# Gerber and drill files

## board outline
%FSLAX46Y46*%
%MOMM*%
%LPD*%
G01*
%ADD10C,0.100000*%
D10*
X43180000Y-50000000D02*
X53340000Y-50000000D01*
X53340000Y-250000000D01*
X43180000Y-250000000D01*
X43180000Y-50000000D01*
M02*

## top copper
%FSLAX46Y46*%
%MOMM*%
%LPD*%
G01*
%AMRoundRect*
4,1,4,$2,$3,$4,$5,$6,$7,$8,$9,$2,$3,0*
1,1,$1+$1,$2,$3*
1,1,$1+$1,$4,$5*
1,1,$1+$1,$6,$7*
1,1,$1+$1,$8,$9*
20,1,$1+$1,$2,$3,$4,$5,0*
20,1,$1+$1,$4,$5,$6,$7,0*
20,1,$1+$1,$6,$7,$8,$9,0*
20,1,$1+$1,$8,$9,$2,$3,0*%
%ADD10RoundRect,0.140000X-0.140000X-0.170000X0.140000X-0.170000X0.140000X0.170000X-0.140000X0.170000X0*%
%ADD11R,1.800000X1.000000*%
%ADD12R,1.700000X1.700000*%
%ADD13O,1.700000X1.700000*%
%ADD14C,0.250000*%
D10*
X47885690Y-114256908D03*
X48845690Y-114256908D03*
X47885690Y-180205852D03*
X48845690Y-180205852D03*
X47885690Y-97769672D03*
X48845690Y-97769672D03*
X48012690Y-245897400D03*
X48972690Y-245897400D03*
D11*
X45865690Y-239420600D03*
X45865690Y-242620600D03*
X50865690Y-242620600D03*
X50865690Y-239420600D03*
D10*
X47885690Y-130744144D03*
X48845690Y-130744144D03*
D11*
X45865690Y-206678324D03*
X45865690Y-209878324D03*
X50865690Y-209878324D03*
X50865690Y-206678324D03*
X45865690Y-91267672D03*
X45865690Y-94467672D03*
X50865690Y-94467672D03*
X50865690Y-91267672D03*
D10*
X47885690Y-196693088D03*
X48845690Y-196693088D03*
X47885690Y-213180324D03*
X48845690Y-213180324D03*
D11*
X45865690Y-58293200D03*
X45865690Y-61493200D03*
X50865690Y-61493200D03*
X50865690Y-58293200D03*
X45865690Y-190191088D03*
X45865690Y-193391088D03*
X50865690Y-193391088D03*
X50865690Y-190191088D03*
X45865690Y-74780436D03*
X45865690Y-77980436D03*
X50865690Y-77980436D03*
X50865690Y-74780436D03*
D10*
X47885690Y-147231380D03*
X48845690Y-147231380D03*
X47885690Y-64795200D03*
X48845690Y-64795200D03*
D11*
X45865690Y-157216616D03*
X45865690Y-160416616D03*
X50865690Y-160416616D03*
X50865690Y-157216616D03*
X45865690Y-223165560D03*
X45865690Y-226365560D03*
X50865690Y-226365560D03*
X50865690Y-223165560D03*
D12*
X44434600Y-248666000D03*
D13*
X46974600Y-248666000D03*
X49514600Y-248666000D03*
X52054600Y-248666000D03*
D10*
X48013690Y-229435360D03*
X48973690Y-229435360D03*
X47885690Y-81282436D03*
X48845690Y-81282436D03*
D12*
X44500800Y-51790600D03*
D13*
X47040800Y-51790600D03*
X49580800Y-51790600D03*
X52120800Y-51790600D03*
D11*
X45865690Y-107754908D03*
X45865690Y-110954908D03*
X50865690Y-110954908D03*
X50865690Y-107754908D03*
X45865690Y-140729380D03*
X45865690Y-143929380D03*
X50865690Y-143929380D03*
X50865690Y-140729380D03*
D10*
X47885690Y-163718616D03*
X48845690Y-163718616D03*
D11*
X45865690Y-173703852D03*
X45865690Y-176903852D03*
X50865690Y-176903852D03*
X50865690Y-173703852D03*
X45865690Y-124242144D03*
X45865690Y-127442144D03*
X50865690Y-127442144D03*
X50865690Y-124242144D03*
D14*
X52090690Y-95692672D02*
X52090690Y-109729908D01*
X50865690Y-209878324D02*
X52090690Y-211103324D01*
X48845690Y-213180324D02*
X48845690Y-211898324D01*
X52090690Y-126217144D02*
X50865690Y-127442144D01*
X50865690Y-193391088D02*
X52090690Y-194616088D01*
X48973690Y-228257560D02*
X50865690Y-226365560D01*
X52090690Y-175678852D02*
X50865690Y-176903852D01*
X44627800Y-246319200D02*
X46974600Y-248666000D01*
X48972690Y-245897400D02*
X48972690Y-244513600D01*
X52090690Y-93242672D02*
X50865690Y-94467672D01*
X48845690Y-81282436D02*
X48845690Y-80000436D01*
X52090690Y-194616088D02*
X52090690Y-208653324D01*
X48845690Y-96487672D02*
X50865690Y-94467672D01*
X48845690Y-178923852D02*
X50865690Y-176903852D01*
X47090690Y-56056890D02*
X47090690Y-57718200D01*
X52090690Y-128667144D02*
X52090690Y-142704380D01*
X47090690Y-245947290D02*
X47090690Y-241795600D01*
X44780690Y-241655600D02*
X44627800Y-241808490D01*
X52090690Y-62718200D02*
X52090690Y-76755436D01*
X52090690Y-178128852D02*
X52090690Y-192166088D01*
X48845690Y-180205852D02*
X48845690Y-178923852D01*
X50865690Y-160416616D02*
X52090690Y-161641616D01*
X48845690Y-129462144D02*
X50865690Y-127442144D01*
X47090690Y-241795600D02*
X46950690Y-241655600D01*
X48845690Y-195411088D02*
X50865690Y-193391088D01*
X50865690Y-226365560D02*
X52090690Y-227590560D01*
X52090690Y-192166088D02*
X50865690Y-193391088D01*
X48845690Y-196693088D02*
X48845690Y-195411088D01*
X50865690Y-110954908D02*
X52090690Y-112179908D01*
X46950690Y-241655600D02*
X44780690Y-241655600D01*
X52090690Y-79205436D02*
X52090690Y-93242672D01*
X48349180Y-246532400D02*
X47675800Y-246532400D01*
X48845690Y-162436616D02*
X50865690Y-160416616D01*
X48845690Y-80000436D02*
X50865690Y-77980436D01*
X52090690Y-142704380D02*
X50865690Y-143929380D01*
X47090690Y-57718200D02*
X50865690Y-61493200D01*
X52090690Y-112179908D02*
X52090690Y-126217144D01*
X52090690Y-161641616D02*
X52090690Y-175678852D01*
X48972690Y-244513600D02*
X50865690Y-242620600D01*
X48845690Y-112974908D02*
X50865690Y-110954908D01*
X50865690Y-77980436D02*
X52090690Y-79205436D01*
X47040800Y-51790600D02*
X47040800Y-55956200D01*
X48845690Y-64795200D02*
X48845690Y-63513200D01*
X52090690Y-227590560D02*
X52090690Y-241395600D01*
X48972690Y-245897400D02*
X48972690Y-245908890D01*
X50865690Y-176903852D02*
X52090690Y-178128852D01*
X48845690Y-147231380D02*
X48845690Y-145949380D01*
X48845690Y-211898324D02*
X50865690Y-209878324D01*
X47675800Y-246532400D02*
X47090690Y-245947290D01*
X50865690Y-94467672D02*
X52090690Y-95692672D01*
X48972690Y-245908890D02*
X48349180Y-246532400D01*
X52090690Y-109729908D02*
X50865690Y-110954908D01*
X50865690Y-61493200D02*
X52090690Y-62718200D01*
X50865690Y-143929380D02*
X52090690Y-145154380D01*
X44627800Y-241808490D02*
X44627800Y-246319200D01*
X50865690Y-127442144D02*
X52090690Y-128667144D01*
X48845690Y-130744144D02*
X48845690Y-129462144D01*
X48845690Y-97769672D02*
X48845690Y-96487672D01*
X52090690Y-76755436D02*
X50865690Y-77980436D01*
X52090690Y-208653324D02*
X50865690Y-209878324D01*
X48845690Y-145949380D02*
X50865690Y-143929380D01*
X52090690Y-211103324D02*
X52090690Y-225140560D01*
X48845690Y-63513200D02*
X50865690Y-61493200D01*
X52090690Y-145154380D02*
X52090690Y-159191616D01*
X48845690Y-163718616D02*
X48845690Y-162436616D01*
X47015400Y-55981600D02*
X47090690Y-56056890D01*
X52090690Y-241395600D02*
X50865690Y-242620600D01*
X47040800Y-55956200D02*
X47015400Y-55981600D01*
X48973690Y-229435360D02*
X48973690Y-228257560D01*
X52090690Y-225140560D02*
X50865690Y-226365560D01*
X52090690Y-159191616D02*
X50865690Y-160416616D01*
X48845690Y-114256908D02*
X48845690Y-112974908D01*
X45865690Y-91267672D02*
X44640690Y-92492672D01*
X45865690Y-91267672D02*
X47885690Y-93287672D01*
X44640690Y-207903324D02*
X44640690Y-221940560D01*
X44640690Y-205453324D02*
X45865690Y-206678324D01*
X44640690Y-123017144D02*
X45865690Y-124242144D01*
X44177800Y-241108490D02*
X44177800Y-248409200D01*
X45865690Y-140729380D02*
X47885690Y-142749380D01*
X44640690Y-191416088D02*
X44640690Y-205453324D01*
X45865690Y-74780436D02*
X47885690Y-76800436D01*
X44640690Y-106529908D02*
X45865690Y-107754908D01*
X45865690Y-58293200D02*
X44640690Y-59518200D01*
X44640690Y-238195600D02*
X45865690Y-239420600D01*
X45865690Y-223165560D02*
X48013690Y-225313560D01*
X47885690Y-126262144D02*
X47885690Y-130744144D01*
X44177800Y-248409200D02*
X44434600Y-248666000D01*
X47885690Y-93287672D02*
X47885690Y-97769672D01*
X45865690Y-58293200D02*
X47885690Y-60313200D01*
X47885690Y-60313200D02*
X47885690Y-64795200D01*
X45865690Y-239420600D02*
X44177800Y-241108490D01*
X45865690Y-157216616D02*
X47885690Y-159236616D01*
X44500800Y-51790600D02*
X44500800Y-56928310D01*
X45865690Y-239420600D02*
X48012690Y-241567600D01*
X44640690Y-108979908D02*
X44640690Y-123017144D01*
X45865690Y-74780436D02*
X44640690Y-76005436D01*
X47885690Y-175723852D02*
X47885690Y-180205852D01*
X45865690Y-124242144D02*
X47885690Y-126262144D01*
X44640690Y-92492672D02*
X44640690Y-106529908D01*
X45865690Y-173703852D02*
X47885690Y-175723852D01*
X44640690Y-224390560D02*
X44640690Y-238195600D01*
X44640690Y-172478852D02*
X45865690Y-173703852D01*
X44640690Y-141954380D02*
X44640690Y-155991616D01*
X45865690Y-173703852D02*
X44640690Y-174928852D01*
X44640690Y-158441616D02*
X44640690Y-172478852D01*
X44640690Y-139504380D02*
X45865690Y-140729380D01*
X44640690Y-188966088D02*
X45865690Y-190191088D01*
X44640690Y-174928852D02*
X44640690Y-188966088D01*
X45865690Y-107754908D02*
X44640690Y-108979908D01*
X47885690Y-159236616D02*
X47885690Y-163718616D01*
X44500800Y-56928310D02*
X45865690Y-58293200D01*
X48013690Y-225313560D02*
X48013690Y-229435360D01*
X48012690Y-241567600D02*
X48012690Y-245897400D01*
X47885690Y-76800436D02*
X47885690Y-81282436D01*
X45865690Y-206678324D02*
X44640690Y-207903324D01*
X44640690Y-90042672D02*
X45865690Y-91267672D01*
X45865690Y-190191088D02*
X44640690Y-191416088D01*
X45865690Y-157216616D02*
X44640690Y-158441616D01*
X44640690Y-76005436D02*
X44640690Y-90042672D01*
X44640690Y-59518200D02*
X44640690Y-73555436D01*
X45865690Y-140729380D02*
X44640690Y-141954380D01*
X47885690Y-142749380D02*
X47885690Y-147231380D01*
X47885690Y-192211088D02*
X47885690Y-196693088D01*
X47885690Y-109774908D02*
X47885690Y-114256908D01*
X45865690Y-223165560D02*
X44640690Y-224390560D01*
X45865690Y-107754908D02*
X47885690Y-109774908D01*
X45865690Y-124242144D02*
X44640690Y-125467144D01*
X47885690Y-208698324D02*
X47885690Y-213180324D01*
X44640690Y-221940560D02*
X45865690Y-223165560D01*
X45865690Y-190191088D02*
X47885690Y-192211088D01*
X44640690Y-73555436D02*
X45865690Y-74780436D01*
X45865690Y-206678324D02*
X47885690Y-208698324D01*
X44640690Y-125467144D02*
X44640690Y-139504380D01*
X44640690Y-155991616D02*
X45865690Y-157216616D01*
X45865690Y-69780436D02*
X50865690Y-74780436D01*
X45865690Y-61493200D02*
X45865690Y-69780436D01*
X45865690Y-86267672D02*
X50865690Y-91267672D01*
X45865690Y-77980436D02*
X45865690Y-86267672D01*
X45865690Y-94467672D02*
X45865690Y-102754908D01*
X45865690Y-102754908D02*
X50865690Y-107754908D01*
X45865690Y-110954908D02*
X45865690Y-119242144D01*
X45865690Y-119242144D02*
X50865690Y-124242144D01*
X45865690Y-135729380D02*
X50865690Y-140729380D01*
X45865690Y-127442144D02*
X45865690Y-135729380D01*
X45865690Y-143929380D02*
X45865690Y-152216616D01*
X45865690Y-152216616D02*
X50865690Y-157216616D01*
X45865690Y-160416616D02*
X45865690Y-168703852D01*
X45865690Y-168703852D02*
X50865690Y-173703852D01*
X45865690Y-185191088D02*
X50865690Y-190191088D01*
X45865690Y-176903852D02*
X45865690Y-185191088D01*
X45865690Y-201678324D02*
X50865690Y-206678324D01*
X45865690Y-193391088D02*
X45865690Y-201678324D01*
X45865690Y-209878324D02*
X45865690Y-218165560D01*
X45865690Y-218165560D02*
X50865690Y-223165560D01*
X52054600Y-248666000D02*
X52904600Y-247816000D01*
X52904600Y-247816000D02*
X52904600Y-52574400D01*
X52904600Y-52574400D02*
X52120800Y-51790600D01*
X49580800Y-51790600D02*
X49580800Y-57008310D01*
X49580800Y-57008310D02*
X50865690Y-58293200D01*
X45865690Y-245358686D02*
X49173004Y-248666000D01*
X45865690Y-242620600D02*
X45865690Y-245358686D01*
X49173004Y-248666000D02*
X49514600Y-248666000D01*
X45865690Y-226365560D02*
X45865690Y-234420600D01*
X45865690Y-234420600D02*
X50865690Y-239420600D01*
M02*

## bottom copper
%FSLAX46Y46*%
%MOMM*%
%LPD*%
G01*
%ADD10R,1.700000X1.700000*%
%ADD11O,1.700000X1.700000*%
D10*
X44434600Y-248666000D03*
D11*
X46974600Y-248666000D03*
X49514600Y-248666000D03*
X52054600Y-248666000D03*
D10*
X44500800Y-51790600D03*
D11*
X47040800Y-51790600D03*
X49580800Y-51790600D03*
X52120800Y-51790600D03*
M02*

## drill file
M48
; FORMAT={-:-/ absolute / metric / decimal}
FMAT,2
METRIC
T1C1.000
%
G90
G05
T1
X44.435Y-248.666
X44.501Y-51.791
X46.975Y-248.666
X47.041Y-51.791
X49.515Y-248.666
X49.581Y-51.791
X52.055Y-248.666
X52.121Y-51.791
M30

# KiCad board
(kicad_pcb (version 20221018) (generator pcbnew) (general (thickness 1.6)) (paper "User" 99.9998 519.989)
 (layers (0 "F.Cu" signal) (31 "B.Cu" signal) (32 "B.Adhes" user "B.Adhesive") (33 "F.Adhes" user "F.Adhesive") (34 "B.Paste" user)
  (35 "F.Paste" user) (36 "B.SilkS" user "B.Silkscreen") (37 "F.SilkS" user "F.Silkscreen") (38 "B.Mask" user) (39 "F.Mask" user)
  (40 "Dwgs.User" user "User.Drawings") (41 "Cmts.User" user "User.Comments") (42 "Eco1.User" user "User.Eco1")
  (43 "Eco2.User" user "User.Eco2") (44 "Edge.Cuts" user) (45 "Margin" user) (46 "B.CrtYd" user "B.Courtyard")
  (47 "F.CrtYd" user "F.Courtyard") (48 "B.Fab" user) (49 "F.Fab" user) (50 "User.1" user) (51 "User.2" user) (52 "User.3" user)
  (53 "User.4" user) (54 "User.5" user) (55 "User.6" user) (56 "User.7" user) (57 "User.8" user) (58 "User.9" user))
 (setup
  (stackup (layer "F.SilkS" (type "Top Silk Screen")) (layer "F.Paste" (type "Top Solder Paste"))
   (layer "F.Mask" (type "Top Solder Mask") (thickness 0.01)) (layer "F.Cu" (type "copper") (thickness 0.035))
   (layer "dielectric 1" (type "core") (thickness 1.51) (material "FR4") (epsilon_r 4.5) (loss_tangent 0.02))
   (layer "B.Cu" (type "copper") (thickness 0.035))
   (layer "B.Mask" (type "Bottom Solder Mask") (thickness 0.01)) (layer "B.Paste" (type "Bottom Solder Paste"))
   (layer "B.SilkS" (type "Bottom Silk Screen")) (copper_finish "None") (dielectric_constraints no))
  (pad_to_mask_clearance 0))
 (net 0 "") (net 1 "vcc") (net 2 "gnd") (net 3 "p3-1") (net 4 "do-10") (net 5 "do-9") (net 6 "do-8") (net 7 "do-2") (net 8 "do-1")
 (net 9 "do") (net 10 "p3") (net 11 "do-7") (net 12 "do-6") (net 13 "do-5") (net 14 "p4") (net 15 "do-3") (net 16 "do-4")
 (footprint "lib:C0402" (layer "F.Cu") (at 48.36569 114.256908)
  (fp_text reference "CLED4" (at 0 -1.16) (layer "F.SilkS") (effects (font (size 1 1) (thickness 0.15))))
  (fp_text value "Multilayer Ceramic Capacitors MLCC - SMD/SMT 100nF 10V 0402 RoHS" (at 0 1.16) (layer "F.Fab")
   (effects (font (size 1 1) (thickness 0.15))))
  (pad "1" smd roundrect (at -0.48 0) (size 0.56 0.62) (layers "F.Cu" "F.Paste" "F.Mask") (roundrect_rratio 0.25) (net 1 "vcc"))
  (pad "2" smd roundrect (at 0.48 0) (size 0.56 0.62) (layers "F.Cu" "F.Paste" "F.Mask") (roundrect_rratio 0.25) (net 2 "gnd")))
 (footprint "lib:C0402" (layer "F.Cu") (at 48.36569 180.205852)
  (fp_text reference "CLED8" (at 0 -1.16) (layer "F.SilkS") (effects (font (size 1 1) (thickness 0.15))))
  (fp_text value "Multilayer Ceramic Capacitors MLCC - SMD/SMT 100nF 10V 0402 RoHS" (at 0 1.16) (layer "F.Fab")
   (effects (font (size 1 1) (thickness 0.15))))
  (pad "1" smd roundrect (at -0.48 0) (size 0.56 0.62) (layers "F.Cu" "F.Paste" "F.Mask") (roundrect_rratio 0.25) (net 1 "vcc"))
  (pad "2" smd roundrect (at 0.48 0) (size 0.56 0.62) (layers "F.Cu" "F.Paste" "F.Mask") (roundrect_rratio 0.25) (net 2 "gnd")))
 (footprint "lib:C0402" (layer "F.Cu") (at 48.36569 97.769672)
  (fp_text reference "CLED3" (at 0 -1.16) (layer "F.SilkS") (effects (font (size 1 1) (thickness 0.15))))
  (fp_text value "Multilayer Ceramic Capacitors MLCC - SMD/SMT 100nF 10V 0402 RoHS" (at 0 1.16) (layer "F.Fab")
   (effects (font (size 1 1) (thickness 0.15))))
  (pad "1" smd roundrect (at -0.48 0) (size 0.56 0.62) (layers "F.Cu" "F.Paste" "F.Mask") (roundrect_rratio 0.25) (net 1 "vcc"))
  (pad "2" smd roundrect (at 0.48 0) (size 0.56 0.62) (layers "F.Cu" "F.Paste" "F.Mask") (roundrect_rratio 0.25) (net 2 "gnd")))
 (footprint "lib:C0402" (layer "F.Cu") (at 48.49269 245.8974)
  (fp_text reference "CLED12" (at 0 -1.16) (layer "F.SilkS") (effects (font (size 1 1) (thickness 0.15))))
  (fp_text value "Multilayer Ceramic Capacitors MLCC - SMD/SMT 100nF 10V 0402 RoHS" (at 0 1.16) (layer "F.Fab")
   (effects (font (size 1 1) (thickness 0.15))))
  (pad "1" smd roundrect (at -0.48 0) (size 0.56 0.62) (layers "F.Cu" "F.Paste" "F.Mask") (roundrect_rratio 0.25) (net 1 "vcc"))
  (pad "2" smd roundrect (at 0.48 0) (size 0.56 0.62) (layers "F.Cu" "F.Paste" "F.Mask") (roundrect_rratio 0.25) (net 2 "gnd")))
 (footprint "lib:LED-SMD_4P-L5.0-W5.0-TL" (layer "F.Cu") (at 48.36569 241.0206)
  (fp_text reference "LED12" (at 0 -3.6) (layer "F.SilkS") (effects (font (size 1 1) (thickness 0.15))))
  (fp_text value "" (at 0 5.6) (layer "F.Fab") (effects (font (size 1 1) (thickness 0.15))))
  (pad "1" smd rect (at -2.5 -1.6 180) (size 1.8 1) (layers "F.Cu" "F.Paste" "F.Mask") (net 1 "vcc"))
  (pad "2" smd rect (at -2.5 1.6 180) (size 1.8 1) (layers "F.Cu" "F.Paste" "F.Mask") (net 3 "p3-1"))
  (pad "3" smd rect (at 2.5 1.6 180) (size 1.8 1) (layers "F.Cu" "F.Paste" "F.Mask") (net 2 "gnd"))
  (pad "4" smd rect (at 2.5 -1.6 180) (size 1.8 1) (layers "F.Cu" "F.Paste" "F.Mask") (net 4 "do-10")))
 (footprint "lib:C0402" (layer "F.Cu") (at 48.36569 130.744144)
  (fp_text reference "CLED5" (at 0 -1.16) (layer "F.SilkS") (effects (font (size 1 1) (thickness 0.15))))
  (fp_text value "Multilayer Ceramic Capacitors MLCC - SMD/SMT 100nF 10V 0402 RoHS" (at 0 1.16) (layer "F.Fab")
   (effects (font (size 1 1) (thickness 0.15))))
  (pad "1" smd roundrect (at -0.48 0) (size 0.56 0.62) (layers "F.Cu" "F.Paste" "F.Mask") (roundrect_rratio 0.25) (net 1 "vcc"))
  (pad "2" smd roundrect (at 0.48 0) (size 0.56 0.62) (layers "F.Cu" "F.Paste" "F.Mask") (roundrect_rratio 0.25) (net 2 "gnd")))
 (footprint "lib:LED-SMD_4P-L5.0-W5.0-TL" (layer "F.Cu") (at 48.36569 208.278324)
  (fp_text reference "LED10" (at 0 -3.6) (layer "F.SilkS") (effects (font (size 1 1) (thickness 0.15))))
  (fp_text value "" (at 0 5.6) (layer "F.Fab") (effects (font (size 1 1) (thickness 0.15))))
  (pad "1" smd rect (at -2.5 -1.6 180) (size 1.8 1) (layers "F.Cu" "F.Paste" "F.Mask") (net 1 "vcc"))
  (pad "2" smd rect (at -2.5 1.6 180) (size 1.8 1) (layers "F.Cu" "F.Paste" "F.Mask") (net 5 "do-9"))
  (pad "3" smd rect (at 2.5 1.6 180) (size 1.8 1) (layers "F.Cu" "F.Paste" "F.Mask") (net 2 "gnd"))
  (pad "4" smd rect (at 2.5 -1.6 180) (size 1.8 1) (layers "F.Cu" "F.Paste" "F.Mask") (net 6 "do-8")))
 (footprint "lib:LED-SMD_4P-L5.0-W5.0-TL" (layer "F.Cu") (at 48.36569 92.867672)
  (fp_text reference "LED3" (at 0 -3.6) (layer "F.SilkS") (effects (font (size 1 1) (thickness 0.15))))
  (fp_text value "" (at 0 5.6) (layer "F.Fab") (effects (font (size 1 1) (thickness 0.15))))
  (pad "1" smd rect (at -2.5 -1.6 180) (size 1.8 1) (layers "F.Cu" "F.Paste" "F.Mask") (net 1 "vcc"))
  (pad "2" smd rect (at -2.5 1.6 180) (size 1.8 1) (layers "F.Cu" "F.Paste" "F.Mask") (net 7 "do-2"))
  (pad "3" smd rect (at 2.5 1.6 180) (size 1.8 1) (layers "F.Cu" "F.Paste" "F.Mask") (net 2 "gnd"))
  (pad "4" smd rect (at 2.5 -1.6 180) (size 1.8 1) (layers "F.Cu" "F.Paste" "F.Mask") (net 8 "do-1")))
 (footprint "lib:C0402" (layer "F.Cu") (at 48.36569 196.693088)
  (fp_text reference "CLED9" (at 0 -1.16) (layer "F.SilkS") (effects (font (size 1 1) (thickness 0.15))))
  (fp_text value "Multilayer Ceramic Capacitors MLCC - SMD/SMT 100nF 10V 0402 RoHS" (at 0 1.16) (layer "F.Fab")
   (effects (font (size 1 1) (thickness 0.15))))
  (pad "1" smd roundrect (at -0.48 0) (size 0.56 0.62) (layers "F.Cu" "F.Paste" "F.Mask") (roundrect_rratio 0.25) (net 1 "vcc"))
  (pad "2" smd roundrect (at 0.48 0) (size 0.56 0.62) (layers "F.Cu" "F.Paste" "F.Mask") (roundrect_rratio 0.25) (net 2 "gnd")))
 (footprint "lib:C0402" (layer "F.Cu") (at 48.36569 213.180324)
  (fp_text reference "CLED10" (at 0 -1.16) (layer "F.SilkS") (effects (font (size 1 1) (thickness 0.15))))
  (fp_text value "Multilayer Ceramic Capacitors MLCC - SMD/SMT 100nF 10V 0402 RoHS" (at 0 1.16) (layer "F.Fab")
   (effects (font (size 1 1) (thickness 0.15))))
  (pad "1" smd roundrect (at -0.48 0) (size 0.56 0.62) (layers "F.Cu" "F.Paste" "F.Mask") (roundrect_rratio 0.25) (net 1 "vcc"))
  (pad "2" smd roundrect (at 0.48 0) (size 0.56 0.62) (layers "F.Cu" "F.Paste" "F.Mask") (roundrect_rratio 0.25) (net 2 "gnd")))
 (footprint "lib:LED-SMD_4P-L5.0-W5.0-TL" (layer "F.Cu") (at 48.36569 59.8932)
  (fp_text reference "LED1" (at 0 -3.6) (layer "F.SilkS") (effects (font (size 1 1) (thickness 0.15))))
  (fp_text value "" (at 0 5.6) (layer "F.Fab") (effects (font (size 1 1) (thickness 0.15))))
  (pad "1" smd rect (at -2.5 -1.6 180) (size 1.8 1) (layers "F.Cu" "F.Paste" "F.Mask") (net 1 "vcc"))
  (pad "2" smd rect (at -2.5 1.6 180) (size 1.8 1) (layers "F.Cu" "F.Paste" "F.Mask") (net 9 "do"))
  (pad "3" smd rect (at 2.5 1.6 180) (size 1.8 1) (layers "F.Cu" "F.Paste" "F.Mask") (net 2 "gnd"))
  (pad "4" smd rect (at 2.5 -1.6 180) (size 1.8 1) (layers "F.Cu" "F.Paste" "F.Mask") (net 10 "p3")))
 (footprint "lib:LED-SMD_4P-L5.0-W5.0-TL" (layer "F.Cu") (at 48.36569 191.791088)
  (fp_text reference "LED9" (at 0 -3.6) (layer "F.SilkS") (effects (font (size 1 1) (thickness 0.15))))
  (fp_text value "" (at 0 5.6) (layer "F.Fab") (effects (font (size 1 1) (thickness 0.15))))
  (pad "1" smd rect (at -2.5 -1.6 180) (size 1.8 1) (layers "F.Cu" "F.Paste" "F.Mask") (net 1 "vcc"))
  (pad "2" smd rect (at -2.5 1.6 180) (size 1.8 1) (layers "F.Cu" "F.Paste" "F.Mask") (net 6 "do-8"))
  (pad "3" smd rect (at 2.5 1.6 180) (size 1.8 1) (layers "F.Cu" "F.Paste" "F.Mask") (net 2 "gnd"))
  (pad "4" smd rect (at 2.5 -1.6 180) (size 1.8 1) (layers "F.Cu" "F.Paste" "F.Mask") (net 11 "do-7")))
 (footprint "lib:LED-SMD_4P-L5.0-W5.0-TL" (layer "F.Cu") (at 48.36569 76.380436)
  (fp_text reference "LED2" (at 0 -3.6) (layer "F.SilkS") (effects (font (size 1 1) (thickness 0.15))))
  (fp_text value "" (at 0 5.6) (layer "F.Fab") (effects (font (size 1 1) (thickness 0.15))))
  (pad "1" smd rect (at -2.5 -1.6 180) (size 1.8 1) (layers "F.Cu" "F.Paste" "F.Mask") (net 1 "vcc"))
  (pad "2" smd rect (at -2.5 1.6 180) (size 1.8 1) (layers "F.Cu" "F.Paste" "F.Mask") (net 8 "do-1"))
  (pad "3" smd rect (at 2.5 1.6 180) (size 1.8 1) (layers "F.Cu" "F.Paste" "F.Mask") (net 2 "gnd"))
  (pad "4" smd rect (at 2.5 -1.6 180) (size 1.8 1) (layers "F.Cu" "F.Paste" "F.Mask") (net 9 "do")))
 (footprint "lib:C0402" (layer "F.Cu") (at 48.36569 147.23138)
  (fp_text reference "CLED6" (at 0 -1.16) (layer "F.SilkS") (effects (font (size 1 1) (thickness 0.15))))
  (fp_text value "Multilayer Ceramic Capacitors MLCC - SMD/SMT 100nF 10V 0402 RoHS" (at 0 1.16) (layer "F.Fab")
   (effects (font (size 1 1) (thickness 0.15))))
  (pad "1" smd roundrect (at -0.48 0) (size 0.56 0.62) (layers "F.Cu" "F.Paste" "F.Mask") (roundrect_rratio 0.25) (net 1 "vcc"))
  (pad "2" smd roundrect (at 0.48 0) (size 0.56 0.62) (layers "F.Cu" "F.Paste" "F.Mask") (roundrect_rratio 0.25) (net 2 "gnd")))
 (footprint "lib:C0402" (layer "F.Cu") (at 48.36569 64.7952)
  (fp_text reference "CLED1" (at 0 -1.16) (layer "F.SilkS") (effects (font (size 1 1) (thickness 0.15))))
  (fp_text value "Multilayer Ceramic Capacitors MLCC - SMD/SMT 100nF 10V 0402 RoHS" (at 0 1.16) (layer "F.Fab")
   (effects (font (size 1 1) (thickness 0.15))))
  (pad "1" smd roundrect (at -0.48 0) (size 0.56 0.62) (layers "F.Cu" "F.Paste" "F.Mask") (roundrect_rratio 0.25) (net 1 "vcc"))
  (pad "2" smd roundrect (at 0.48 0) (size 0.56 0.62) (layers "F.Cu" "F.Paste" "F.Mask") (roundrect_rratio 0.25) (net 2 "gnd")))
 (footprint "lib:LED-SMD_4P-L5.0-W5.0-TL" (layer "F.Cu") (at 48.36569 158.816616)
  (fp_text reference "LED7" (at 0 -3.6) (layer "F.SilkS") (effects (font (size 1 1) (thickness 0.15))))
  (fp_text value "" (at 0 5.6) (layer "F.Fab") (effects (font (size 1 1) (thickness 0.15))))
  (pad "1" smd rect (at -2.5 -1.6 180) (size 1.8 1) (layers "F.Cu" "F.Paste" "F.Mask") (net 1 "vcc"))
  (pad "2" smd rect (at -2.5 1.6 180) (size 1.8 1) (layers "F.Cu" "F.Paste" "F.Mask") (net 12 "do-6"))
  (pad "3" smd rect (at 2.5 1.6 180) (size 1.8 1) (layers "F.Cu" "F.Paste" "F.Mask") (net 2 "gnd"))
  (pad "4" smd rect (at 2.5 -1.6 180) (size 1.8 1) (layers "F.Cu" "F.Paste" "F.Mask") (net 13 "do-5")))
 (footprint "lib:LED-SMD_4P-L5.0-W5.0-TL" (layer "F.Cu") (at 48.36569 224.76556)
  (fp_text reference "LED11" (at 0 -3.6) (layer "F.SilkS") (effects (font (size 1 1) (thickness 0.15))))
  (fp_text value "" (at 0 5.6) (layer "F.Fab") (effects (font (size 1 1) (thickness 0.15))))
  (pad "1" smd rect (at -2.5 -1.6 180) (size 1.8 1) (layers "F.Cu" "F.Paste" "F.Mask") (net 1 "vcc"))
  (pad "2" smd rect (at -2.5 1.6 180) (size 1.8 1) (layers "F.Cu" "F.Paste" "F.Mask") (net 4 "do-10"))
  (pad "3" smd rect (at 2.5 1.6 180) (size 1.8 1) (layers "F.Cu" "F.Paste" "F.Mask") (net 2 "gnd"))
  (pad "4" smd rect (at 2.5 -1.6 180) (size 1.8 1) (layers "F.Cu" "F.Paste" "F.Mask") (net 5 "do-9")))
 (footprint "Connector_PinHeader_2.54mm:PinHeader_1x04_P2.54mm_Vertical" (layer "F.Cu") (at 44.4346 248.666 90)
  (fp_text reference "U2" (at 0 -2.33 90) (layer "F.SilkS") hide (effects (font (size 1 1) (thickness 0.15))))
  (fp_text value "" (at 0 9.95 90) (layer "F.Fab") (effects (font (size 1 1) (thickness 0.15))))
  (pad "1" thru_hole rect (at 0 0 90) (size 1.7 1.7) (drill 1) (layers "*.Cu" "*.Mask") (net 1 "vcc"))
  (pad "2" thru_hole oval (at 0 2.54 90) (size 1.7 1.7) (drill 1) (layers "*.Cu" "*.Mask") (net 2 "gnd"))
  (pad "3" thru_hole oval (at 0 5.08 90) (size 1.7 1.7) (drill 1) (layers "*.Cu" "*.Mask") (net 3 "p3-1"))
  (pad "4" thru_hole oval (at 0 7.62 90) (size 1.7 1.7) (drill 1) (layers "*.Cu" "*.Mask") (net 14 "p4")))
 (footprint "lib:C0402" (layer "F.Cu") (at 48.49369 229.43536)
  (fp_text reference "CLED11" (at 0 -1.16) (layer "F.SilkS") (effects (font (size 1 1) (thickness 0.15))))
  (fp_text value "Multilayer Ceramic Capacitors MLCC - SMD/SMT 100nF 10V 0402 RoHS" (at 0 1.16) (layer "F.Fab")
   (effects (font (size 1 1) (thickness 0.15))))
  (pad "1" smd roundrect (at -0.48 0) (size 0.56 0.62) (layers "F.Cu" "F.Paste" "F.Mask") (roundrect_rratio 0.25) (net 1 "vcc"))
  (pad "2" smd roundrect (at 0.48 0) (size 0.56 0.62) (layers "F.Cu" "F.Paste" "F.Mask") (roundrect_rratio 0.25) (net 2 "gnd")))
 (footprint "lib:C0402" (layer "F.Cu") (at 48.36569 81.282436)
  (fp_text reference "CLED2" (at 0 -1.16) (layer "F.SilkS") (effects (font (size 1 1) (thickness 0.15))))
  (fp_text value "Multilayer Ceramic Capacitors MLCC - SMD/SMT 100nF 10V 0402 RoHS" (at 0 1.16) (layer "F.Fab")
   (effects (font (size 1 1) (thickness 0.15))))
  (pad "1" smd roundrect (at -0.48 0) (size 0.56 0.62) (layers "F.Cu" "F.Paste" "F.Mask") (roundrect_rratio 0.25) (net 1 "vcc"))
  (pad "2" smd roundrect (at 0.48 0) (size 0.56 0.62) (layers "F.Cu" "F.Paste" "F.Mask") (roundrect_rratio 0.25) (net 2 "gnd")))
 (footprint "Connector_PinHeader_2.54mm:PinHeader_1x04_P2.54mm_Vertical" (layer "F.Cu") (at 44.5008 51.7906 90)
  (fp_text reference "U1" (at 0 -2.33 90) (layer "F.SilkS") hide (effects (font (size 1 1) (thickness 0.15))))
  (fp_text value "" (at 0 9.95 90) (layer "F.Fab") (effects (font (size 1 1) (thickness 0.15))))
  (pad "1" thru_hole rect (at 0 0 90) (size 1.7 1.7) (drill 1) (layers "*.Cu" "*.Mask") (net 1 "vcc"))
  (pad "2" thru_hole oval (at 0 2.54 90) (size 1.7 1.7) (drill 1) (layers "*.Cu" "*.Mask") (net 2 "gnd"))
  (pad "3" thru_hole oval (at 0 5.08 90) (size 1.7 1.7) (drill 1) (layers "*.Cu" "*.Mask") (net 10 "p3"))
  (pad "4" thru_hole oval (at 0 7.62 90) (size 1.7 1.7) (drill 1) (layers "*.Cu" "*.Mask") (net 14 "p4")))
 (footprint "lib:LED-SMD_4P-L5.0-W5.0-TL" (layer "F.Cu") (at 48.36569 109.354908)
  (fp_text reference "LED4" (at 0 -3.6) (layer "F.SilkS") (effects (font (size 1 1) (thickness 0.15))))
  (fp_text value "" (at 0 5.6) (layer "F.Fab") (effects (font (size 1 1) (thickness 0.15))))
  (pad "1" smd rect (at -2.5 -1.6 180) (size 1.8 1) (layers "F.Cu" "F.Paste" "F.Mask") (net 1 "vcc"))
  (pad "2" smd rect (at -2.5 1.6 180) (size 1.8 1) (layers "F.Cu" "F.Paste" "F.Mask") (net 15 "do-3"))
  (pad "3" smd rect (at 2.5 1.6 180) (size 1.8 1) (layers "F.Cu" "F.Paste" "F.Mask") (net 2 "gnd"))
  (pad "4" smd rect (at 2.5 -1.6 180) (size 1.8 1) (layers "F.Cu" "F.Paste" "F.Mask") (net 7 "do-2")))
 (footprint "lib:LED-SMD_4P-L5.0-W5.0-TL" (layer "F.Cu") (at 48.36569 142.32938)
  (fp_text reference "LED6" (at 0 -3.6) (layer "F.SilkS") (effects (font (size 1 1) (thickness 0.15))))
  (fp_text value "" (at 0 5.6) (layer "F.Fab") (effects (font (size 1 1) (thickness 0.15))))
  (pad "1" smd rect (at -2.5 -1.6 180) (size 1.8 1) (layers "F.Cu" "F.Paste" "F.Mask") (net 1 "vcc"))
  (pad "2" smd rect (at -2.5 1.6 180) (size 1.8 1) (layers "F.Cu" "F.Paste" "F.Mask") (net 13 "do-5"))
  (pad "3" smd rect (at 2.5 1.6 180) (size 1.8 1) (layers "F.Cu" "F.Paste" "F.Mask") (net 2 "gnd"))
  (pad "4" smd rect (at 2.5 -1.6 180) (size 1.8 1) (layers "F.Cu" "F.Paste" "F.Mask") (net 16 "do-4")))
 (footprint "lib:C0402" (layer "F.Cu") (at 48.36569 163.718616)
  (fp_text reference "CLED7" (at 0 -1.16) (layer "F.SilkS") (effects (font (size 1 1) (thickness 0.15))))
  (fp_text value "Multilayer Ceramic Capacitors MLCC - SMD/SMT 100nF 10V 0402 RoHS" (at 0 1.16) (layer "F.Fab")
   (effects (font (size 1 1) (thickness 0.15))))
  (pad "1" smd roundrect (at -0.48 0) (size 0.56 0.62) (layers "F.Cu" "F.Paste" "F.Mask") (roundrect_rratio 0.25) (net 1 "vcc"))
  (pad "2" smd roundrect (at 0.48 0) (size 0.56 0.62) (layers "F.Cu" "F.Paste" "F.Mask") (roundrect_rratio 0.25) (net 2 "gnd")))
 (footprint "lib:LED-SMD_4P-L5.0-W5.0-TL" (layer "F.Cu") (at 48.36569 175.303852)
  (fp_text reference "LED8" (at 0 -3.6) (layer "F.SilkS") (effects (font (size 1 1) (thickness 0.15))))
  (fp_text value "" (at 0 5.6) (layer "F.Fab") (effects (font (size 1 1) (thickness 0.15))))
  (pad "1" smd rect (at -2.5 -1.6 180) (size 1.8 1) (layers "F.Cu" "F.Paste" "F.Mask") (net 1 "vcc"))
  (pad "2" smd rect (at -2.5 1.6 180) (size 1.8 1) (layers "F.Cu" "F.Paste" "F.Mask") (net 11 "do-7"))
  (pad "3" smd rect (at 2.5 1.6 180) (size 1.8 1) (layers "F.Cu" "F.Paste" "F.Mask") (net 2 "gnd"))
  (pad "4" smd rect (at 2.5 -1.6 180) (size 1.8 1) (layers "F.Cu" "F.Paste" "F.Mask") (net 12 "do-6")))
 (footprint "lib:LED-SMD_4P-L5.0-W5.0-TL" (layer "F.Cu") (at 48.36569 125.842144)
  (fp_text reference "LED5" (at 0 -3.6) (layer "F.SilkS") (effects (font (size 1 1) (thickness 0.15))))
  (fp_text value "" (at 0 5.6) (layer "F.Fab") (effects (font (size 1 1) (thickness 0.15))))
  (pad "1" smd rect (at -2.5 -1.6 180) (size 1.8 1) (layers "F.Cu" "F.Paste" "F.Mask") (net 1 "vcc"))
  (pad "2" smd rect (at -2.5 1.6 180) (size 1.8 1) (layers "F.Cu" "F.Paste" "F.Mask") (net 16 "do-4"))
  (pad "3" smd rect (at 2.5 1.6 180) (size 1.8 1) (layers "F.Cu" "F.Paste" "F.Mask") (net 2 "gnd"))
  (pad "4" smd rect (at 2.5 -1.6 180) (size 1.8 1) (layers "F.Cu" "F.Paste" "F.Mask") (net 15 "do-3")))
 (gr_rect (start 43.18 50) (end 53.34 250) (stroke (width 0.1) (type default)) (fill none) (layer "Edge.Cuts"))
 (segment (start 52.09069 95.692672) (end 52.09069 109.729908) (width 0.25) (layer "F.Cu") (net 2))
 (segment (start 50.86569 209.878324) (end 52.09069 211.103324) (width 0.25) (layer "F.Cu") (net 2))
 (segment (start 48.84569 213.180324) (end 48.84569 211.898324) (width 0.25) (layer "F.Cu") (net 2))
 (segment (start 52.09069 126.217144) (end 50.86569 127.442144) (width 0.25) (layer "F.Cu") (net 2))
 (segment (start 50.86569 193.391088) (end 52.09069 194.616088) (width 0.25) (layer "F.Cu") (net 2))
 (segment (start 48.97369 228.25756) (end 50.86569 226.36556) (width 0.25) (layer "F.Cu") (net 2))
 (segment (start 52.09069 175.678852) (end 50.86569 176.903852) (width 0.25) (layer "F.Cu") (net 2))
 (segment (start 44.6278 246.3192) (end 46.9746 248.666) (width 0.25) (layer "F.Cu") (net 2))
 (segment (start 48.97269 245.8974) (end 48.97269 244.5136) (width 0.25) (layer "F.Cu") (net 2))
 (segment (start 52.09069 93.242672) (end 50.86569 94.467672) (width 0.25) (layer "F.Cu") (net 2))
 (segment (start 48.84569 81.282436) (end 48.84569 80.000436) (width 0.25) (layer "F.Cu") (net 2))
 (segment (start 52.09069 194.616088) (end 52.09069 208.653324) (width 0.25) (layer "F.Cu") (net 2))
 (segment (start 48.84569 96.487672) (end 50.86569 94.467672) (width 0.25) (layer "F.Cu") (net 2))
 (segment (start 48.84569 178.923852) (end 50.86569 176.903852) (width 0.25) (layer "F.Cu") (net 2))
 (segment (start 47.09069 56.05689) (end 47.09069 57.7182) (width 0.25) (layer "F.Cu") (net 2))
 (segment (start 52.09069 128.667144) (end 52.09069 142.70438) (width 0.25) (layer "F.Cu") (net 2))
 (segment (start 47.09069 245.94729) (end 47.09069 241.7956) (width 0.25) (layer "F.Cu") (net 2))
 (segment (start 44.78069 241.6556) (end 44.6278 241.80849) (width 0.25) (layer "F.Cu") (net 2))
 (segment (start 52.09069 62.7182) (end 52.09069 76.755436) (width 0.25) (layer "F.Cu") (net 2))
 (segment (start 52.09069 178.128852) (end 52.09069 192.166088) (width 0.25) (layer "F.Cu") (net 2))
 (segment (start 48.84569 180.205852) (end 48.84569 178.923852) (width 0.25) (layer "F.Cu") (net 2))
 (segment (start 50.86569 160.416616) (end 52.09069 161.641616) (width 0.25) (layer "F.Cu") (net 2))
 (segment (start 48.84569 129.462144) (end 50.86569 127.442144) (width 0.25) (layer "F.Cu") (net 2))
 (segment (start 47.09069 241.7956) (end 46.95069 241.6556) (width 0.25) (layer "F.Cu") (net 2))
 (segment (start 48.84569 195.411088) (end 50.86569 193.391088) (width 0.25) (layer "F.Cu") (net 2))
 (segment (start 50.86569 226.36556) (end 52.09069 227.59056) (width 0.25) (layer "F.Cu") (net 2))
 (segment (start 52.09069 192.166088) (end 50.86569 193.391088) (width 0.25) (layer "F.Cu") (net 2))
 (segment (start 48.84569 196.693088) (end 48.84569 195.411088) (width 0.25) (layer "F.Cu") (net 2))
 (segment (start 50.86569 110.954908) (end 52.09069 112.179908) (width 0.25) (layer "F.Cu") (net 2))
 (segment (start 46.95069 241.6556) (end 44.78069 241.6556) (width 0.25) (layer "F.Cu") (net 2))
 (segment (start 52.09069 79.205436) (end 52.09069 93.242672) (width 0.25) (layer "F.Cu") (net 2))
 (segment (start 48.34918 246.5324) (end 47.6758 246.5324) (width 0.25) (layer "F.Cu") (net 2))
 (segment (start 48.84569 162.436616) (end 50.86569 160.416616) (width 0.25) (layer "F.Cu") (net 2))
 (segment (start 48.84569 80.000436) (end 50.86569 77.980436) (width 0.25) (layer "F.Cu") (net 2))
 (segment (start 52.09069 142.70438) (end 50.86569 143.92938) (width 0.25) (layer "F.Cu") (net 2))
 (segment (start 47.09069 57.7182) (end 50.86569 61.4932) (width 0.25) (layer "F.Cu") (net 2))
 (segment (start 52.09069 112.179908) (end 52.09069 126.217144) (width 0.25) (layer "F.Cu") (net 2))
 (segment (start 52.09069 161.641616) (end 52.09069 175.678852) (width 0.25) (layer "F.Cu") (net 2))
 (segment (start 48.97269 244.5136) (end 50.86569 242.6206) (width 0.25) (layer "F.Cu") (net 2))
 (segment (start 48.84569 112.974908) (end 50.86569 110.954908) (width 0.25) (layer "F.Cu") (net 2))
 (segment (start 50.86569 77.980436) (end 52.09069 79.205436) (width 0.25) (layer "F.Cu") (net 2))
 (segment (start 47.0408 51.7906) (end 47.0408 55.9562) (width 0.25) (layer "F.Cu") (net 2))
 (segment (start 48.84569 64.7952) (end 48.84569 63.5132) (width 0.25) (layer "F.Cu") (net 2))
 (segment (start 52.09069 227.59056) (end 52.09069 241.3956) (width 0.25) (layer "F.Cu") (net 2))
 (segment (start 48.97269 245.8974) (end 48.97269 245.90889) (width 0.25) (layer "F.Cu") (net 2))
 (segment (start 50.86569 176.903852) (end 52.09069 178.128852) (width 0.25) (layer "F.Cu") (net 2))
 (segment (start 48.84569 147.23138) (end 48.84569 145.94938) (width 0.25) (layer "F.Cu") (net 2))
 (segment (start 48.84569 211.898324) (end 50.86569 209.878324) (width 0.25) (layer "F.Cu") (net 2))
 (segment (start 47.6758 246.5324) (end 47.09069 245.94729) (width 0.25) (layer "F.Cu") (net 2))
 (segment (start 50.86569 94.467672) (end 52.09069 95.692672) (width 0.25) (layer "F.Cu") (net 2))
 (segment (start 48.97269 245.90889) (end 48.34918 246.5324) (width 0.25) (layer "F.Cu") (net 2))
 (segment (start 52.09069 109.729908) (end 50.86569 110.954908) (width 0.25) (layer "F.Cu") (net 2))
 (segment (start 50.86569 61.4932) (end 52.09069 62.7182) (width 0.25) (layer "F.Cu") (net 2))
 (segment (start 50.86569 143.92938) (end 52.09069 145.15438) (width 0.25) (layer "F.Cu") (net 2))
 (segment (start 44.6278 241.80849) (end 44.6278 246.3192) (width 0.25) (layer "F.Cu") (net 2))
 (segment (start 50.86569 127.442144) (end 52.09069 128.667144) (width 0.25) (layer "F.Cu") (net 2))
 (segment (start 48.84569 130.744144) (end 48.84569 129.462144) (width 0.25) (layer "F.Cu") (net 2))
 (segment (start 48.84569 97.769672) (end 48.84569 96.487672) (width 0.25) (layer "F.Cu") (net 2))
 (segment (start 52.09069 76.755436) (end 50.86569 77.980436) (width 0.25) (layer "F.Cu") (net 2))
 (segment (start 52.09069 208.653324) (end 50.86569 209.878324) (width 0.25) (layer "F.Cu") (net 2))
 (segment (start 48.84569 145.94938) (end 50.86569 143.92938) (width 0.25) (layer "F.Cu") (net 2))
 (segment (start 52.09069 211.103324) (end 52.09069 225.14056) (width 0.25) (layer "F.Cu") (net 2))
 (segment (start 48.84569 63.5132) (end 50.86569 61.4932) (width 0.25) (layer "F.Cu") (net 2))
 (segment (start 52.09069 145.15438) (end 52.09069 159.191616) (width 0.25) (layer "F.Cu") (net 2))
 (segment (start 48.84569 163.718616) (end 48.84569 162.436616) (width 0.25) (layer "F.Cu") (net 2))
 (segment (start 47.0154 55.9816) (end 47.09069 56.05689) (width 0.25) (layer "F.Cu") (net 2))
 (segment (start 52.09069 241.3956) (end 50.86569 242.6206) (width 0.25) (layer "F.Cu") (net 2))
 (segment (start 47.0408 55.9562) (end 47.0154 55.9816) (width 0.25) (layer "F.Cu") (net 2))
 (segment (start 48.97369 229.43536) (end 48.97369 228.25756) (width 0.25) (layer "F.Cu") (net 2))
 (segment (start 52.09069 225.14056) (end 50.86569 226.36556) (width 0.25) (layer "F.Cu") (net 2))
 (segment (start 52.09069 159.191616) (end 50.86569 160.416616) (width 0.25) (layer "F.Cu") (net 2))
 (segment (start 48.84569 114.256908) (end 48.84569 112.974908) (width 0.25) (layer "F.Cu") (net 2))
 (segment (start 45.86569 91.267672) (end 44.64069 92.492672) (width 0.25) (layer "F.Cu") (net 1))
 (segment (start 45.86569 91.267672) (end 47.88569 93.287672) (width 0.25) (layer "F.Cu") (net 1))
 (segment (start 44.64069 207.903324) (end 44.64069 221.94056) (width 0.25) (layer "F.Cu") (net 1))
 (segment (start 44.64069 205.453324) (end 45.86569 206.678324) (width 0.25) (layer "F.Cu") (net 1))
 (segment (start 44.64069 123.017144) (end 45.86569 124.242144) (width 0.25) (layer "F.Cu") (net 1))
 (segment (start 44.1778 241.10849) (end 44.1778 248.4092) (width 0.25) (layer "F.Cu") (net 1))
 (segment (start 45.86569 140.72938) (end 47.88569 142.74938) (width 0.25) (layer "F.Cu") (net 1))
 (segment (start 44.64069 191.416088) (end 44.64069 205.453324) (width 0.25) (layer "F.Cu") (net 1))
 (segment (start 45.86569 74.780436) (end 47.88569 76.800436) (width 0.25) (layer "F.Cu") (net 1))
 (segment (start 44.64069 106.529908) (end 45.86569 107.754908) (width 0.25) (layer "F.Cu") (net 1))
 (segment (start 45.86569 58.2932) (end 44.64069 59.5182) (width 0.25) (layer "F.Cu") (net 1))
 (segment (start 44.64069 238.1956) (end 45.86569 239.4206) (width 0.25) (layer "F.Cu") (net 1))
 (segment (start 45.86569 223.16556) (end 48.01369 225.31356) (width 0.25) (layer "F.Cu") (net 1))
 (segment (start 47.88569 126.262144) (end 47.88569 130.744144) (width 0.25) (layer "F.Cu") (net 1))
 (segment (start 44.1778 248.4092) (end 44.4346 248.666) (width 0.25) (layer "F.Cu") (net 1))
 (segment (start 47.88569 93.287672) (end 47.88569 97.769672) (width 0.25) (layer "F.Cu") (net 1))
 (segment (start 45.86569 58.2932) (end 47.88569 60.3132) (width 0.25) (layer "F.Cu") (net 1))
 (segment (start 47.88569 60.3132) (end 47.88569 64.7952) (width 0.25) (layer "F.Cu") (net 1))
 (segment (start 45.86569 239.4206) (end 44.1778 241.10849) (width 0.25) (layer "F.Cu") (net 1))
 (segment (start 45.86569 157.216616) (end 47.88569 159.236616) (width 0.25) (layer "F.Cu") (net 1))
 (segment (start 44.5008 51.7906) (end 44.5008 56.92831) (width 0.25) (layer "F.Cu") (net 1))
 (segment (start 45.86569 239.4206) (end 48.01269 241.5676) (width 0.25) (layer "F.Cu") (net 1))
 (segment (start 44.64069 108.979908) (end 44.64069 123.017144) (width 0.25) (layer "F.Cu") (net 1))
 (segment (start 45.86569 74.780436) (end 44.64069 76.005436) (width 0.25) (layer "F.Cu") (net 1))
 (segment (start 47.88569 175.723852) (end 47.88569 180.205852) (width 0.25) (layer "F.Cu") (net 1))
 (segment (start 45.86569 124.242144) (end 47.88569 126.262144) (width 0.25) (layer "F.Cu") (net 1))
 (segment (start 44.64069 92.492672) (end 44.64069 106.529908) (width 0.25) (layer "F.Cu") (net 1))
 (segment (start 45.86569 173.703852) (end 47.88569 175.723852) (width 0.25) (layer "F.Cu") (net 1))
 (segment (start 44.64069 224.39056) (end 44.64069 238.1956) (width 0.25) (layer "F.Cu") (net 1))
 (segment (start 44.64069 172.478852) (end 45.86569 173.703852) (width 0.25) (layer "F.Cu") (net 1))
 (segment (start 44.64069 141.95438) (end 44.64069 155.991616) (width 0.25) (layer "F.Cu") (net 1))
 (segment (start 45.86569 173.703852) (end 44.64069 174.928852) (width 0.25) (layer "F.Cu") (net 1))
 (segment (start 44.64069 158.441616) (end 44.64069 172.478852) (width 0.25) (layer "F.Cu") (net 1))
 (segment (start 44.64069 139.50438) (end 45.86569 140.72938) (width 0.25) (layer "F.Cu") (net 1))
 (segment (start 44.64069 188.966088) (end 45.86569 190.191088) (width 0.25) (layer "F.Cu") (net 1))
 (segment (start 44.64069 174.928852) (end 44.64069 188.966088) (width 0.25) (layer "F.Cu") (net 1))
 (segment (start 45.86569 107.754908) (end 44.64069 108.979908) (width 0.25) (layer "F.Cu") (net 1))
 (segment (start 47.88569 159.236616) (end 47.88569 163.718616) (width 0.25) (layer "F.Cu") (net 1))
 (segment (start 44.5008 56.92831) (end 45.86569 58.2932) (width 0.25) (layer "F.Cu") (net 1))
 (segment (start 48.01369 225.31356) (end 48.01369 229.43536) (width 0.25) (layer "F.Cu") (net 1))
 (segment (start 48.01269 241.5676) (end 48.01269 245.8974) (width 0.25) (layer "F.Cu") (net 1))
 (segment (start 47.88569 76.800436) (end 47.88569 81.282436) (width 0.25) (layer "F.Cu") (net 1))
 (segment (start 45.86569 206.678324) (end 44.64069 207.903324) (width 0.25) (layer "F.Cu") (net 1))
 (segment (start 44.64069 90.042672) (end 45.86569 91.267672) (width 0.25) (layer "F.Cu") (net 1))
 (segment (start 45.86569 190.191088) (end 44.64069 191.416088) (width 0.25) (layer "F.Cu") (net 1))
 (segment (start 45.86569 157.216616) (end 44.64069 158.441616) (width 0.25) (layer "F.Cu") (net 1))
 (segment (start 44.64069 76.005436) (end 44.64069 90.042672) (width 0.25) (layer "F.Cu") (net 1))
 (segment (start 44.64069 59.5182) (end 44.64069 73.555436) (width 0.25) (layer "F.Cu") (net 1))
 (segment (start 45.86569 140.72938) (end 44.64069 141.95438) (width 0.25) (layer "F.Cu") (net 1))
 (segment (start 47.88569 142.74938) (end 47.88569 147.23138) (width 0.25) (layer "F.Cu") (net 1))
 (segment (start 47.88569 192.211088) (end 47.88569 196.693088) (width 0.25) (layer "F.Cu") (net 1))
 (segment (start 47.88569 109.774908) (end 47.88569 114.256908) (width 0.25) (layer "F.Cu") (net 1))
 (segment (start 45.86569 223.16556) (end 44.64069 224.39056) (width 0.25) (layer "F.Cu") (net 1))
 (segment (start 45.86569 107.754908) (end 47.88569 109.774908) (width 0.25) (layer "F.Cu") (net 1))
 (segment (start 45.86569 124.242144) (end 44.64069 125.467144) (width 0.25) (layer "F.Cu") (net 1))
 (segment (start 47.88569 208.698324) (end 47.88569 213.180324) (width 0.25) (layer "F.Cu") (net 1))
 (segment (start 44.64069 221.94056) (end 45.86569 223.16556) (width 0.25) (layer "F.Cu") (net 1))
 (segment (start 45.86569 190.191088) (end 47.88569 192.211088) (width 0.25) (layer "F.Cu") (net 1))
 (segment (start 44.64069 73.555436) (end 45.86569 74.780436) (width 0.25) (layer "F.Cu") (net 1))
 (segment (start 45.86569 206.678324) (end 47.88569 208.698324) (width 0.25) (layer "F.Cu") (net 1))
 (segment (start 44.64069 125.467144) (end 44.64069 139.50438) (width 0.25) (layer "F.Cu") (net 1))
 (segment (start 44.64069 155.991616) (end 45.86569 157.216616) (width 0.25) (layer "F.Cu") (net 1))
 (segment (start 45.86569 69.780436) (end 50.86569 74.780436) (width 0.25) (layer "F.Cu") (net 9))
 (segment (start 45.86569 61.4932) (end 45.86569 69.780436) (width 0.25) (layer "F.Cu") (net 9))
 (segment (start 45.86569 86.267672) (end 50.86569 91.267672) (width 0.25) (layer "F.Cu") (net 8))
 (segment (start 45.86569 77.980436) (end 45.86569 86.267672) (width 0.25) (layer "F.Cu") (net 8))
 (segment (start 45.86569 94.467672) (end 45.86569 102.754908) (width 0.25) (layer "F.Cu") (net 7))
 (segment (start 45.86569 102.754908) (end 50.86569 107.754908) (width 0.25) (layer "F.Cu") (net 7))
 (segment (start 45.86569 110.954908) (end 45.86569 119.242144) (width 0.25) (layer "F.Cu") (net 15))
 (segment (start 45.86569 119.242144) (end 50.86569 124.242144) (width 0.25) (layer "F.Cu") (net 15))
 (segment (start 45.86569 135.72938) (end 50.86569 140.72938) (width 0.25) (layer "F.Cu") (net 16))
 (segment (start 45.86569 127.442144) (end 45.86569 135.72938) (width 0.25) (layer "F.Cu") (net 16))
 (segment (start 45.86569 143.92938) (end 45.86569 152.216616) (width 0.25) (layer "F.Cu") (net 13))
 (segment (start 45.86569 152.216616) (end 50.86569 157.216616) (width 0.25) (layer "F.Cu") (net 13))
 (segment (start 45.86569 160.416616) (end 45.86569 168.703852) (width 0.25) (layer "F.Cu") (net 12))
 (segment (start 45.86569 168.703852) (end 50.86569 173.703852) (width 0.25) (layer "F.Cu") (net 12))
 (segment (start 45.86569 185.191088) (end 50.86569 190.191088) (width 0.25) (layer "F.Cu") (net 11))
 (segment (start 45.86569 176.903852) (end 45.86569 185.191088) (width 0.25) (layer "F.Cu") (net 11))
 (segment (start 45.86569 201.678324) (end 50.86569 206.678324) (width 0.25) (layer "F.Cu") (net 6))
 (segment (start 45.86569 193.391088) (end 45.86569 201.678324) (width 0.25) (layer "F.Cu") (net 6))
 (segment (start 45.86569 209.878324) (end 45.86569 218.16556) (width 0.25) (layer "F.Cu") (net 5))
 (segment (start 45.86569 218.16556) (end 50.86569 223.16556) (width 0.25) (layer "F.Cu") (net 5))
 (segment (start 52.0546 248.666) (end 52.9046 247.816) (width 0.25) (layer "F.Cu") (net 14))
 (segment (start 52.9046 247.816) (end 52.9046 52.5744) (width 0.25) (layer "F.Cu") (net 14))
 (segment (start 52.9046 52.5744) (end 52.1208 51.7906) (width 0.25) (layer "F.Cu") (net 14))
 (segment (start 49.5808 51.7906) (end 49.5808 57.00831) (width 0.25) (layer "F.Cu") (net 10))
 (segment (start 49.5808 57.00831) (end 50.86569 58.2932) (width 0.25) (layer "F.Cu") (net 10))
 (segment (start 45.86569 245.358686) (end 49.173004 248.666) (width 0.25) (layer "F.Cu") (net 3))
 (segment (start 45.86569 242.6206) (end 45.86569 245.358686) (width 0.25) (layer "F.Cu") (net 3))
 (segment (start 49.173004 248.666) (end 49.5146 248.666) (width 0.25) (layer "F.Cu") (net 3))
 (segment (start 45.86569 226.36556) (end 45.86569 234.4206) (width 0.25) (layer "F.Cu") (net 4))
 (segment (start 45.86569 234.4206) (end 50.86569 239.4206) (width 0.25) (layer "F.Cu") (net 4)))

